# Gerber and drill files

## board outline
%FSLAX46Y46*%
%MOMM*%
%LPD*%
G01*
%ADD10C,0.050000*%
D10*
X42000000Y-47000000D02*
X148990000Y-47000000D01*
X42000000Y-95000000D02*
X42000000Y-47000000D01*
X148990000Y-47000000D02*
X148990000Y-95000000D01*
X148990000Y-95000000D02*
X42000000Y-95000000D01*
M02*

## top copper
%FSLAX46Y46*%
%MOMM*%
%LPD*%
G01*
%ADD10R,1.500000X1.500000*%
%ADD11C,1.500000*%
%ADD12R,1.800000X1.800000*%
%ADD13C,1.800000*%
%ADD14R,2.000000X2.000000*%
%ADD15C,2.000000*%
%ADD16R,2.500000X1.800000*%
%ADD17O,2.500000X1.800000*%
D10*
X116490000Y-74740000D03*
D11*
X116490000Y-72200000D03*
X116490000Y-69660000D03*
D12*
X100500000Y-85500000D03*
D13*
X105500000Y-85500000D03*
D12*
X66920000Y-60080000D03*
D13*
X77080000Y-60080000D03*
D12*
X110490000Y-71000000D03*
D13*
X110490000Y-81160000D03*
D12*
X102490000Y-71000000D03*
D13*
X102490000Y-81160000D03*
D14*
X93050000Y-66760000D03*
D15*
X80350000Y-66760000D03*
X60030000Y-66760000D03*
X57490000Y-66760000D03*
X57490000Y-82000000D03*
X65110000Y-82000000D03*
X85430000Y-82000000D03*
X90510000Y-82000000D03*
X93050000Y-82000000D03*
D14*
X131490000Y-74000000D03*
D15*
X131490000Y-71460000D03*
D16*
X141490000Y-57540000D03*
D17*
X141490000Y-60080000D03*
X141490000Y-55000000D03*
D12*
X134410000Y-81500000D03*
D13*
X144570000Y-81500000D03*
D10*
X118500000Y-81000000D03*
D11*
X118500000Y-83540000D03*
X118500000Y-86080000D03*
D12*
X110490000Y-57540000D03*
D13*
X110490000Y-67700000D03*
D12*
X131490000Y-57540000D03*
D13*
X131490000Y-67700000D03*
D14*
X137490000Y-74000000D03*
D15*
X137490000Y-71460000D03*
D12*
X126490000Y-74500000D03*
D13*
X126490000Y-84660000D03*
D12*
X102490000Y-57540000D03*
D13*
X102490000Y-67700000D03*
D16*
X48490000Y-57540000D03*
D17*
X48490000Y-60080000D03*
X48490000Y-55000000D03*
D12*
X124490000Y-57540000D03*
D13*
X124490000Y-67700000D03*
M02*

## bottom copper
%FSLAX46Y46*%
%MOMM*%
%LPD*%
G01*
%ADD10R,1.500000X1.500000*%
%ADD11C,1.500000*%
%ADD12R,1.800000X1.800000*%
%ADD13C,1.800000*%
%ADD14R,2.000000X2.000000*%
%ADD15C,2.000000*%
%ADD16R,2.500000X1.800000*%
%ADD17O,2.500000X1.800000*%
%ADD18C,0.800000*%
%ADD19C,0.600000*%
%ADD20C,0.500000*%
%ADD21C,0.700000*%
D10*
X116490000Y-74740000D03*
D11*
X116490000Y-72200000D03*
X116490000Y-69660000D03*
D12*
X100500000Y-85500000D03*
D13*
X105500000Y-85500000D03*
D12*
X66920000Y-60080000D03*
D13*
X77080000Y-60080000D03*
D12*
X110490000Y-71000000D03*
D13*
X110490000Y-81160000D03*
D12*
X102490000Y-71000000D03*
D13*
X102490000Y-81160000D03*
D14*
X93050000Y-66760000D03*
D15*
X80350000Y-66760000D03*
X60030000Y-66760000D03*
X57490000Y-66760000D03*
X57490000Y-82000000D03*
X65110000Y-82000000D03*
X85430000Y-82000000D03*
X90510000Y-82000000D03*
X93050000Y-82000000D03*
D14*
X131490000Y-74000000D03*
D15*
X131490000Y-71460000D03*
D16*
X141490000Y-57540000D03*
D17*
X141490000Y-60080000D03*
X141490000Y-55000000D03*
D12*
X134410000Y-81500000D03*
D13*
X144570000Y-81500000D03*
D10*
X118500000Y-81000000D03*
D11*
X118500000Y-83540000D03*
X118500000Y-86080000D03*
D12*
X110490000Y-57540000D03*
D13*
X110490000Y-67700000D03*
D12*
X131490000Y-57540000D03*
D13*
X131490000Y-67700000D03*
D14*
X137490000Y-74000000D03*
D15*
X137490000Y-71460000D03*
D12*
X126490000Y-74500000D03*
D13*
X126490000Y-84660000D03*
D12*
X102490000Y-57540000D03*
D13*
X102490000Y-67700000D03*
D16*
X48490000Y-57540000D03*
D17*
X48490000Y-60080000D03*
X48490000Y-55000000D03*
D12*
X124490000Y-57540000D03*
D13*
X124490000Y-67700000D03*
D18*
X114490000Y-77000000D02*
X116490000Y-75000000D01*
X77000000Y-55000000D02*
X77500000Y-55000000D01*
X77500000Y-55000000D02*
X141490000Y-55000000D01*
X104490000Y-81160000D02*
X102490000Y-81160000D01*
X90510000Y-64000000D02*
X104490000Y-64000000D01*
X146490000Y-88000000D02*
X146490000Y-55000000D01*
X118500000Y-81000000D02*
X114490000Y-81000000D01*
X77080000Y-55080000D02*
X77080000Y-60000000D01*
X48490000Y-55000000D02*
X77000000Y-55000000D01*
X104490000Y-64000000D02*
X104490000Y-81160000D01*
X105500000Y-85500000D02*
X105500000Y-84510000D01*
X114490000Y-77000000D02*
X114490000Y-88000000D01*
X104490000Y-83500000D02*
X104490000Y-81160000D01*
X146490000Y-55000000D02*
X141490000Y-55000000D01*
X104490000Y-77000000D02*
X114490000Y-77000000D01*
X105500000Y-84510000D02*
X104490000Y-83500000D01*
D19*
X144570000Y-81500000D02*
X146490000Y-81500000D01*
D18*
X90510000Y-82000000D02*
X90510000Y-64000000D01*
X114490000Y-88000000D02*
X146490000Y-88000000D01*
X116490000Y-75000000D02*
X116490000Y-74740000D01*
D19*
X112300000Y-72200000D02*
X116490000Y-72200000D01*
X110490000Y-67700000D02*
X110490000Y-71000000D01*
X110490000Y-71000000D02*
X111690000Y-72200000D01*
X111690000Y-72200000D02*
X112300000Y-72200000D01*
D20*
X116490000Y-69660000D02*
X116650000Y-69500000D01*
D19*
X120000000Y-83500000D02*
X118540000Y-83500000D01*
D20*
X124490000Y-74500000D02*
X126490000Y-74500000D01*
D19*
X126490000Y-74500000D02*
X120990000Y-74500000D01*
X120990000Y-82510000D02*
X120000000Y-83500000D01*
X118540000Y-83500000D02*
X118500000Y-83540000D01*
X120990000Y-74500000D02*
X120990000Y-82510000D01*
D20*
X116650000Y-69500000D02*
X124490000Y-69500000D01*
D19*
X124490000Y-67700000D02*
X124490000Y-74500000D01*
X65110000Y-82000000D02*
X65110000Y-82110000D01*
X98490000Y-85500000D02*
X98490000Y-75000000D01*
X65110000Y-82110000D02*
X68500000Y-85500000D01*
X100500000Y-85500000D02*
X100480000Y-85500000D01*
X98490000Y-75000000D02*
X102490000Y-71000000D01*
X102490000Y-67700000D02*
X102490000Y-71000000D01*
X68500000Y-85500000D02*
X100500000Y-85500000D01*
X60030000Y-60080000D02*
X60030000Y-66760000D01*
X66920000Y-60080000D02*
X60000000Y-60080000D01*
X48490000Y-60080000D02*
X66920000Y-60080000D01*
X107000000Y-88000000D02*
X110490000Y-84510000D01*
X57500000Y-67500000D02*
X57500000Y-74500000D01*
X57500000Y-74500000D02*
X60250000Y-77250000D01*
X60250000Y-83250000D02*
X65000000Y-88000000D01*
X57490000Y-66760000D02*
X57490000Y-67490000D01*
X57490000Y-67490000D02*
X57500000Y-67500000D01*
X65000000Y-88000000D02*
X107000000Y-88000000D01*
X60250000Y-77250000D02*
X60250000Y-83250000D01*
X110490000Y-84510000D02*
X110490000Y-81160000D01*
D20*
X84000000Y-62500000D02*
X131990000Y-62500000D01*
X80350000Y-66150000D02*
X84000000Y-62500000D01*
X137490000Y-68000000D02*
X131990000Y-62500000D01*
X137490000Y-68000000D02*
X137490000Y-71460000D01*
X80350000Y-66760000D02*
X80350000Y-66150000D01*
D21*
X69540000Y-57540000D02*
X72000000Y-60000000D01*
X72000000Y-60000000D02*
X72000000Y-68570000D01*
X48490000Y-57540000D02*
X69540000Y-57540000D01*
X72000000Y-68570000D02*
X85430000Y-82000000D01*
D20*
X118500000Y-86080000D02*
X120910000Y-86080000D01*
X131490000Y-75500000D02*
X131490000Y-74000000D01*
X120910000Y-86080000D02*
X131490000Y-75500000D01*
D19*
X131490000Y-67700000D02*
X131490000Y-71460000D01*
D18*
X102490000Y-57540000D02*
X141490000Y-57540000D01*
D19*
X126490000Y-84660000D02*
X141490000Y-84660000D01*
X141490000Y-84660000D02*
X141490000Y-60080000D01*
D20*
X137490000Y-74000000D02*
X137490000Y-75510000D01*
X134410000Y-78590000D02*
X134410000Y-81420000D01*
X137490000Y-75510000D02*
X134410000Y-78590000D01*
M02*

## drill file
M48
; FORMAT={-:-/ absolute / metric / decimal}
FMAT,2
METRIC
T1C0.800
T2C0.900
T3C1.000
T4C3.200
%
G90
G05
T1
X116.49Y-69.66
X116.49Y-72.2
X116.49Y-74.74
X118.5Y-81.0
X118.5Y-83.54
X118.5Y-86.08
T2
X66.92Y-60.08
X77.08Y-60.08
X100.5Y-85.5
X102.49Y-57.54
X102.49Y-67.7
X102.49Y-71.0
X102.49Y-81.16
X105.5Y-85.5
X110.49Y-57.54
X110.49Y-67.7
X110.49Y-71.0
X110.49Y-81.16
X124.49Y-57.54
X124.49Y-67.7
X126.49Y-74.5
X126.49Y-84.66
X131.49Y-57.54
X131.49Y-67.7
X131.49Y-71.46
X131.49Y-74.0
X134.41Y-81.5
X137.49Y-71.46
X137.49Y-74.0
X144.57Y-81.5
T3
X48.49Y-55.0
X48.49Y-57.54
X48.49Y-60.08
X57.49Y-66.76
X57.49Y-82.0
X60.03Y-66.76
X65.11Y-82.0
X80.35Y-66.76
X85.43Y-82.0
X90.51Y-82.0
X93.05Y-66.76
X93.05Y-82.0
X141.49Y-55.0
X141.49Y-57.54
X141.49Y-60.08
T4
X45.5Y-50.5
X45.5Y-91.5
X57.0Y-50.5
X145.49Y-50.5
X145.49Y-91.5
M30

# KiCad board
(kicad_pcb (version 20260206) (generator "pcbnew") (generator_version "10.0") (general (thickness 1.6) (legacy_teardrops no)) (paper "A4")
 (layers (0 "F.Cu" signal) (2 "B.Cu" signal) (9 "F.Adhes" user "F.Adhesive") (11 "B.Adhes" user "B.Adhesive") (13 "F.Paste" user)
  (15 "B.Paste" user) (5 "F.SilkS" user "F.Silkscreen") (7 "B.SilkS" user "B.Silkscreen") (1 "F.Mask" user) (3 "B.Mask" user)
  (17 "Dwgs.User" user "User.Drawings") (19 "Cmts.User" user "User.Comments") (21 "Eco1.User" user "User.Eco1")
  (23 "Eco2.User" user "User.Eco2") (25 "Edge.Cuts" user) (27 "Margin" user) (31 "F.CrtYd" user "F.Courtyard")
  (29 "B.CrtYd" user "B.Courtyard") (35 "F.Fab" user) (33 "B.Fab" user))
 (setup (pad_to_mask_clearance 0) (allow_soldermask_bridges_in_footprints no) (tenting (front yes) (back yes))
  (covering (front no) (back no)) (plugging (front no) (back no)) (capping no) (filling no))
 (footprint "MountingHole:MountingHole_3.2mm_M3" (layer "F.Cu") (at 145.49 50.5)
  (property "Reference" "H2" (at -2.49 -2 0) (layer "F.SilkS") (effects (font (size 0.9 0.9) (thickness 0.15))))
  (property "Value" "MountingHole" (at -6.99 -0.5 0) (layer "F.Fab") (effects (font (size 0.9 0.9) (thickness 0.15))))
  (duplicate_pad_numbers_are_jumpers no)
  (pad "" np_thru_hole circle (at 0 0) (size 3.2 3.2) (drill 3.2) (layers "*.Cu" "*.Mask")))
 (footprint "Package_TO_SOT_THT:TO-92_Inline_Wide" (layer "F.Cu") (at 116.49 74.74 90)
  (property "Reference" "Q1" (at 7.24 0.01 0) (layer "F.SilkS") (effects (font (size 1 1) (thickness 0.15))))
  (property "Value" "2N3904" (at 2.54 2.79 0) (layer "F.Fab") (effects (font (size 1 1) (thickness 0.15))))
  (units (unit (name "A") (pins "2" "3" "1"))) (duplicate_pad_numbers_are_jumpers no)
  (pad "1" thru_hole rect (at 0 0) (size 1.5 1.5) (drill 0.8) (layers "*.Cu" "*.Mask") (remove_unused_layers no) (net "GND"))
  (pad "2" thru_hole circle (at 2.54 0) (size 1.5 1.5) (drill 0.8) (layers "*.Cu" "*.Mask") (remove_unused_layers no) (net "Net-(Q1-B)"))
  (pad "3" thru_hole circle (at 5.08 0) (size 1.5 1.5) (drill 0.8) (layers "*.Cu" "*.Mask") (remove_unused_layers no) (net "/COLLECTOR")))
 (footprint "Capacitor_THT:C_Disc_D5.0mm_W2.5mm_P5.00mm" (layer "F.Cu") (at 100.5 85.5)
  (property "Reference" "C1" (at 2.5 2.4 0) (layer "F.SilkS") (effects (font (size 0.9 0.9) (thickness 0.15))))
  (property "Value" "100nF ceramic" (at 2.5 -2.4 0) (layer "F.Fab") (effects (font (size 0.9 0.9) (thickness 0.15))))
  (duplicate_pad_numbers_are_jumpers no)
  (pad "1" thru_hole rect (at 0 0) (size 1.8 1.8) (drill 0.9) (layers "*.Cu" "*.Mask") (remove_unused_layers no) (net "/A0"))
  (pad "2" thru_hole circle (at 5 0) (size 1.8 1.8) (drill 0.9) (layers "*.Cu" "*.Mask") (remove_unused_layers no) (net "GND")))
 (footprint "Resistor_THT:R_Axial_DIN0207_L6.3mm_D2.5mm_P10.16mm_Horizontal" (layer "F.Cu") (at 66.92 60.08)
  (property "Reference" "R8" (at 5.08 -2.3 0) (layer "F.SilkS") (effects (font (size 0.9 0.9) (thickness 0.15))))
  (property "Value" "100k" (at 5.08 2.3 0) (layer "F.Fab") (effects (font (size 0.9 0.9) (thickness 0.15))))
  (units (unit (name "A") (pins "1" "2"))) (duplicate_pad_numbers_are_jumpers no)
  (pad "1" thru_hole rect (at 0 0) (size 1.8 1.8) (drill 0.9) (layers "*.Cu" "*.Mask") (remove_unused_layers no) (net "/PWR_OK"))
  (pad "2" thru_hole circle (at 10.16 0) (size 1.8 1.8) (drill 0.9) (layers "*.Cu" "*.Mask") (remove_unused_layers no) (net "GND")))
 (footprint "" (layer "F.Cu") (at 57 50.5)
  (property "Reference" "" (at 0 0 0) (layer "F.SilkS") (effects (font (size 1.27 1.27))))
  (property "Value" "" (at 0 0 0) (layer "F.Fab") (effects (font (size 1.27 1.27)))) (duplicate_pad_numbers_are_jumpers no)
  (pad "" np_thru_hole circle (at 0 0) (size 3.2 3.2) (drill 3.2) (layers "*.Cu" "*.Mask")))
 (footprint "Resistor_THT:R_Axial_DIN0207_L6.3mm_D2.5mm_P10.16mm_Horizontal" (layer "F.Cu") (at 110.49 71 -90)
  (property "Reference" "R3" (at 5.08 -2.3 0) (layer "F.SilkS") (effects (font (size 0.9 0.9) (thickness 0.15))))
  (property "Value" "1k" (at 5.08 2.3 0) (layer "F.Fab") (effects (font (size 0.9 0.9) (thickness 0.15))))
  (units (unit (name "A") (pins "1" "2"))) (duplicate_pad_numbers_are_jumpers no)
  (pad "1" thru_hole rect (at 0 0) (size 1.8 1.8) (drill 0.9) (layers "*.Cu" "*.Mask") (remove_unused_layers no) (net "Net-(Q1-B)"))
  (pad "2" thru_hole circle (at 10.16 0) (size 1.8 1.8) (drill 0.9) (layers "*.Cu" "*.Mask") (remove_unused_layers no) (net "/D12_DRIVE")))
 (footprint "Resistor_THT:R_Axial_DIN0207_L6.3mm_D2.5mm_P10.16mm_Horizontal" (layer "F.Cu") (at 102.49 71 -90)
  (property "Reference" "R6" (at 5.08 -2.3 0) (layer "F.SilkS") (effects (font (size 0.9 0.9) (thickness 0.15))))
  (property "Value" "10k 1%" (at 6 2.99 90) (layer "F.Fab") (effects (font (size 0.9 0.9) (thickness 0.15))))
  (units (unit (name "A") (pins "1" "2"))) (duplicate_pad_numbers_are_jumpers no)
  (pad "1" thru_hole rect (at 0 0) (size 1.8 1.8) (drill 0.9) (layers "*.Cu" "*.Mask") (remove_unused_layers no) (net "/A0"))
  (pad "2" thru_hole circle (at 10.16 0) (size 1.8 1.8) (drill 0.9) (layers "*.Cu" "*.Mask") (remove_unused_layers no) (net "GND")))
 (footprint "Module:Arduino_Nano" (layer "F.Cu") (at 57.49 82 90)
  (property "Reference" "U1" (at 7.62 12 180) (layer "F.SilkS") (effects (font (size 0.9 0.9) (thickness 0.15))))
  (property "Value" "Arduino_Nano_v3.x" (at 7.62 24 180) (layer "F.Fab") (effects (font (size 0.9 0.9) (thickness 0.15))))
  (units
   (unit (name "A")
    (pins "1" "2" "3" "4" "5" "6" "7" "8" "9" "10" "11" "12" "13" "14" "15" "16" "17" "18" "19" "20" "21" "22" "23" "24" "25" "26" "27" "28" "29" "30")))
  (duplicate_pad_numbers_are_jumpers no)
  (pad "1" thru_hole rect (at 15.24 35.56 180) (size 2 2) (drill 1) (layers "*.Cu" "*.Mask") (remove_unused_layers no))
  (pad "6" thru_hole circle (at 15.24 22.86 180) (size 2 2) (drill 1) (layers "*.Cu" "*.Mask") (remove_unused_layers no) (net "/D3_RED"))
  (pad "14" thru_hole circle (at 15.24 2.54 180) (size 2 2) (drill 1) (layers "*.Cu" "*.Mask") (remove_unused_layers no) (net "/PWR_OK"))
  (pad "15" thru_hole circle (at 15.24 0 180) (size 2 2) (drill 1) (layers "*.Cu" "*.Mask") (remove_unused_layers no) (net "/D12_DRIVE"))
  (pad "16" thru_hole circle (at 0 0 180) (size 2 2) (drill 1) (layers "*.Cu" "*.Mask") (remove_unused_layers no))
  (pad "19" thru_hole circle (at 0 7.62 180) (size 2 2) (drill 1) (layers "*.Cu" "*.Mask") (remove_unused_layers no) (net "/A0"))
  (pad "27" thru_hole circle (at 0 27.94 180) (size 2 2) (drill 1) (layers "*.Cu" "*.Mask") (remove_unused_layers no) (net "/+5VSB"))
  (pad "29" thru_hole circle (at 0 33.02 180) (size 2 2) (drill 1) (layers "*.Cu" "*.Mask") (remove_unused_layers no) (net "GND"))
  (pad "30" thru_hole circle (at 0 35.56 180) (size 2 2) (drill 1) (layers "*.Cu" "*.Mask") (remove_unused_layers no)))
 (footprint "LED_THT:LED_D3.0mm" (layer "F.Cu") (at 131.49 74 90)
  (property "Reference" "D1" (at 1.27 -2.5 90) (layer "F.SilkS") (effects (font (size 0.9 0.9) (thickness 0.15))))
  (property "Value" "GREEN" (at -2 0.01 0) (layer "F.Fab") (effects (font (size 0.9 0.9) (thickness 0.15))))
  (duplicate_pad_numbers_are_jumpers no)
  (pad "1" thru_hole rect (at 0 0 90) (size 2 2) (drill 0.9) (layers "*.Cu" "*.Mask") (remove_unused_layers no) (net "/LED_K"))
  (pad "2" thru_hole circle (at 2.54 0 90) (size 2 2) (drill 0.9) (layers "*.Cu" "*.Mask") (remove_unused_layers no) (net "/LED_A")))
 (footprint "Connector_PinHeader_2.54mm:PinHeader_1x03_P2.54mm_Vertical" (layer "F.Cu") (at 141.49 55)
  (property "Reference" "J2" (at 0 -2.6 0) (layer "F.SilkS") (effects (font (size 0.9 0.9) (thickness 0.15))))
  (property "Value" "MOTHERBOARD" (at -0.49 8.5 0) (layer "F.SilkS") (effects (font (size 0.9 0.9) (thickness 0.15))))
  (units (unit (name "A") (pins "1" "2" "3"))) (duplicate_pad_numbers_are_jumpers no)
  (pad "1" thru_hole rect (at 0 2.54) (size 2.5 1.8) (drill 1) (layers "*.Cu" "*.Mask") (remove_unused_layers no) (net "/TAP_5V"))
  (pad "2" thru_hole oval (at 0 5.08) (size 2.5 1.8) (drill 1) (layers "*.Cu" "*.Mask") (remove_unused_layers no) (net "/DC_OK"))
  (pad "3" thru_hole oval (at 0 0) (size 2.5 1.8) (drill 1) (layers "*.Cu" "*.Mask") (remove_unused_layers no) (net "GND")))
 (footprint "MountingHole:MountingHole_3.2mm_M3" (layer "F.Cu") (at 45.5 91.5)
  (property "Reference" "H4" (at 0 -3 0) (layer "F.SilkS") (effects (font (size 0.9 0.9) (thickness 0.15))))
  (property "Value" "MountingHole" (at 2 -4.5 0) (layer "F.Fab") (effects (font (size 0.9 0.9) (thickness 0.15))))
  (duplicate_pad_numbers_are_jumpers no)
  (pad "" np_thru_hole circle (at 0 0) (size 3.2 3.2) (drill 3.2) (layers "*.Cu" "*.Mask")))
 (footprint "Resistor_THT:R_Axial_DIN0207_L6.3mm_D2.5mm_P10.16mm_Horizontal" (layer "F.Cu") (at 134.41 81.5)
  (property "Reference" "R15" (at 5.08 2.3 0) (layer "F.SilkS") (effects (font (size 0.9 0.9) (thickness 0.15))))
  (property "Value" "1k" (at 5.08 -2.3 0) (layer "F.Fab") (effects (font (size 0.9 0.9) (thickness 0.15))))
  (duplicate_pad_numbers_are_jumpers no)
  (pad "1" thru_hole rect (at 0 0) (size 1.8 1.8) (drill 0.9) (layers "*.Cu" "*.Mask") (remove_unused_layers no) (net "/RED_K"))
  (pad "2" thru_hole circle (at 10.16 0) (size 1.8 1.8) (drill 0.9) (layers "*.Cu" "*.Mask") (remove_unused_layers no) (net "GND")))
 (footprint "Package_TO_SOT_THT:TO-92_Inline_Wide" (layer "F.Cu") (at 118.5 81 -90)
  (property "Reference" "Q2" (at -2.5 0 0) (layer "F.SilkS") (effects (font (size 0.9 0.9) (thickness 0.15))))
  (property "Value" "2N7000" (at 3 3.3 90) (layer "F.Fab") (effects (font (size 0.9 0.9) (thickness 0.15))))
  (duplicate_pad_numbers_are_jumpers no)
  (pad "1" thru_hole rect (at 0 0) (size 1.5 1.5) (drill 0.8) (layers "*.Cu" "*.Mask") (remove_unused_layers no) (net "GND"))
  (pad "2" thru_hole circle (at 2.54 0) (size 1.5 1.5) (drill 0.8) (layers "*.Cu" "*.Mask") (remove_unused_layers no) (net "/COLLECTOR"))
  (pad "3" thru_hole circle (at 5.08 0) (size 1.5 1.5) (drill 0.8) (layers "*.Cu" "*.Mask") (remove_unused_layers no) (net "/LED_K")))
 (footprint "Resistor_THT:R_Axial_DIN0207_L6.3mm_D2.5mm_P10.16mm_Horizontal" (layer "F.Cu") (at 110.49 57.54 -90)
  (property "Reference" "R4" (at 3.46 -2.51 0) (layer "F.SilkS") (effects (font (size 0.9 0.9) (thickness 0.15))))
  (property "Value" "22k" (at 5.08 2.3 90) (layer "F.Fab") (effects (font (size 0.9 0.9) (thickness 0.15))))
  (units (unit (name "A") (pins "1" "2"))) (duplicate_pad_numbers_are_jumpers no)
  (pad "1" thru_hole rect (at 0 0 270) (size 1.8 1.8) (drill 0.9) (layers "*.Cu" "*.Mask") (remove_unused_layers no) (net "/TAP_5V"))
  (pad "2" thru_hole circle (at 10.16 0 270) (size 1.8 1.8) (drill 0.9) (layers "*.Cu" "*.Mask") (remove_unused_layers no)
   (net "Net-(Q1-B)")))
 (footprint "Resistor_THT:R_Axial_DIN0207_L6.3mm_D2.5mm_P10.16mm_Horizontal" (layer "F.Cu") (at 131.49 57.54 -90)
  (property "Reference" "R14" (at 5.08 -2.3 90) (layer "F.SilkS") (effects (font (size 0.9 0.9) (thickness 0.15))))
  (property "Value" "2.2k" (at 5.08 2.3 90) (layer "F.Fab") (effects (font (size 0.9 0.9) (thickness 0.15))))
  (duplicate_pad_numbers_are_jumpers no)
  (pad "1" thru_hole rect (at 0 0 270) (size 1.8 1.8) (drill 0.9) (layers "*.Cu" "*.Mask") (remove_unused_layers no) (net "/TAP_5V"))
  (pad "2" thru_hole circle (at 10.16 0 270) (size 1.8 1.8) (drill 0.9) (layers "*.Cu" "*.Mask") (remove_unused_layers no) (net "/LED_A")))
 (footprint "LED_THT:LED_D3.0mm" (layer "F.Cu") (at 137.49 74 90)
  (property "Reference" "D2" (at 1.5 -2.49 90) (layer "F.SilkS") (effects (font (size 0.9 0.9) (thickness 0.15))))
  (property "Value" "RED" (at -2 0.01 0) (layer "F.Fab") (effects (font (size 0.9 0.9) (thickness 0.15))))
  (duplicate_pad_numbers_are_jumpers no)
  (pad "1" thru_hole rect (at 0 0 90) (size 2 2) (drill 0.9) (layers "*.Cu" "*.Mask") (remove_unused_layers no) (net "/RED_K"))
  (pad "2" thru_hole circle (at 2.54 0 90) (size 2 2) (drill 0.9) (layers "*.Cu" "*.Mask") (remove_unused_layers no) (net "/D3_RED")))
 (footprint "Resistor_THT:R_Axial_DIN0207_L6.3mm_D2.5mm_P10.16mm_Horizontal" (layer "F.Cu") (at 126.49 74.5 -90)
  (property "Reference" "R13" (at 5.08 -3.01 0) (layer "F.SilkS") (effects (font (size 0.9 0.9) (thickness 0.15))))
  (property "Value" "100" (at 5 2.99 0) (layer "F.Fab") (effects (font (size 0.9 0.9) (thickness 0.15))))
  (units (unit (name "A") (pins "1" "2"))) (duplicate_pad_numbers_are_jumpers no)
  (pad "1" thru_hole rect (at 0 0) (size 1.8 1.8) (drill 0.9) (layers "*.Cu" "*.Mask") (remove_unused_layers no) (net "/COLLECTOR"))
  (pad "2" thru_hole circle (at 10.16 0) (size 1.8 1.8) (drill 0.9) (layers "*.Cu" "*.Mask") (remove_unused_layers no) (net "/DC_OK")))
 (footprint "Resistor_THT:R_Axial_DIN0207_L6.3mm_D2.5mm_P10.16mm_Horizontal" (layer "F.Cu") (at 102.49 57.54 -90)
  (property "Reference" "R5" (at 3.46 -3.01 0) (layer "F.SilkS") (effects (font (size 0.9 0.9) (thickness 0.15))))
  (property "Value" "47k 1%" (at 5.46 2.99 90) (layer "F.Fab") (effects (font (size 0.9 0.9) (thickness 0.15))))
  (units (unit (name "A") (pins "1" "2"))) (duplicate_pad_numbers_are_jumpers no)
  (pad "1" thru_hole rect (at 0 0 270) (size 1.8 1.8) (drill 0.9) (layers "*.Cu" "*.Mask") (remove_unused_layers no) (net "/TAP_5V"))
  (pad "2" thru_hole circle (at 10.16 0 270) (size 1.8 1.8) (drill 0.9) (layers "*.Cu" "*.Mask") (remove_unused_layers no) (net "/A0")))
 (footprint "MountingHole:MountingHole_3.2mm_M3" (layer "F.Cu") (at 145.49 91.5)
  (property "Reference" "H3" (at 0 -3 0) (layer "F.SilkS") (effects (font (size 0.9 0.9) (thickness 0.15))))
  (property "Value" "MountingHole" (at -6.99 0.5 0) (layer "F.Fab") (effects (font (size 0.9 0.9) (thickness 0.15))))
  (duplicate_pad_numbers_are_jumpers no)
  (pad "" np_thru_hole circle (at 0 0) (size 3.2 3.2) (drill 3.2) (layers "*.Cu" "*.Mask")))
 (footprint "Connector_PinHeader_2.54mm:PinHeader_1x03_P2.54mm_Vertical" (layer "F.Cu") (at 48.49 55)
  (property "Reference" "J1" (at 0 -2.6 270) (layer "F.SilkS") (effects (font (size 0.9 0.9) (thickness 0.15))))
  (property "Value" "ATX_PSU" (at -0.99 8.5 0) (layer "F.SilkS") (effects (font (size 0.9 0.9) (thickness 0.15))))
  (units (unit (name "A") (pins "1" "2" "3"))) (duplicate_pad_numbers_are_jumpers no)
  (pad "1" thru_hole rect (at 0 2.54) (size 2.5 1.8) (drill 1) (layers "*.Cu" "*.Mask") (remove_unused_layers no) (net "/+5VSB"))
  (pad "2" thru_hole oval (at 0 5.08) (size 2.5 1.8) (drill 1) (layers "*.Cu" "*.Mask") (remove_unused_layers no) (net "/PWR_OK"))
  (pad "3" thru_hole oval (at 0 0) (size 2.5 1.8) (drill 1) (layers "*.Cu" "*.Mask") (remove_unused_layers no) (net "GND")))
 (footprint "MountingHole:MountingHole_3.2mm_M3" (layer "F.Cu") (at 45.5 50.5)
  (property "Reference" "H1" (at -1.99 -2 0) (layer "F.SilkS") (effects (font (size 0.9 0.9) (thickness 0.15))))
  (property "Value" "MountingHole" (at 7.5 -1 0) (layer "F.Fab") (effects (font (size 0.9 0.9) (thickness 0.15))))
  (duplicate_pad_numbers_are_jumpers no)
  (pad "" np_thru_hole circle (at 0 0) (size 3.2 3.2) (drill 3.2) (layers "*.Cu" "*.Mask")))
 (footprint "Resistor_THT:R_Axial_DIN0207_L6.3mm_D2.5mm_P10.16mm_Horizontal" (layer "F.Cu") (at 124.49 57.54 -90)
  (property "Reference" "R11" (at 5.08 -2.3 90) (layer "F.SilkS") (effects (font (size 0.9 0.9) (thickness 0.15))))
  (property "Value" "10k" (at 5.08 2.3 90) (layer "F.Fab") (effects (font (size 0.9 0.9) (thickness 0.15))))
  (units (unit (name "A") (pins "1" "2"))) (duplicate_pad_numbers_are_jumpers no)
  (pad "1" thru_hole rect (at 0 0 270) (size 1.8 1.8) (drill 0.9) (layers "*.Cu" "*.Mask") (remove_unused_layers no) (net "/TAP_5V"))
  (pad "2" thru_hole circle (at 10.16 0 270) (size 1.8 1.8) (drill 0.9) (layers "*.Cu" "*.Mask") (remove_unused_layers no)
   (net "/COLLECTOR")))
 (gr_line (start 42 47) (end 148.99 47) (stroke (width 0.05) (type default)) (layer "Edge.Cuts"))
 (gr_line (start 42 95) (end 42 47) (stroke (width 0.05) (type default)) (layer "Edge.Cuts"))
 (gr_line (start 148.99 47) (end 148.99 95) (stroke (width 0.05) (type default)) (layer "Edge.Cuts"))
 (gr_line (start 148.99 95) (end 42 95) (stroke (width 0.05) (type default)) (layer "Edge.Cuts"))
 (segment (start 114.49 77) (end 116.49 75) (width 0.8) (layer "B.Cu") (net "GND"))
 (segment (start 77 55) (end 77.5 55) (width 0.8) (layer "B.Cu") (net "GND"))
 (segment (start 77.5 55) (end 141.49 55) (width 0.8) (layer "B.Cu") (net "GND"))
 (segment (start 104.49 81.16) (end 102.49 81.16) (width 0.8) (layer "B.Cu") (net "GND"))
 (segment (start 90.51 64) (end 104.49 64) (width 0.8) (layer "B.Cu") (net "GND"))
 (segment (start 146.49 88) (end 146.49 55) (width 0.8) (layer "B.Cu") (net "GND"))
 (segment (start 118.5 81) (end 114.49 81) (width 0.8) (layer "B.Cu") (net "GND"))
 (segment (start 77.08 55.08) (end 77.08 60) (width 0.8) (layer "B.Cu") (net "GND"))
 (segment (start 48.49 55) (end 77 55) (width 0.8) (layer "B.Cu") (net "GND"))
 (segment (start 104.49 64) (end 104.49 81.16) (width 0.8) (layer "B.Cu") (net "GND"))
 (segment (start 105.5 85.5) (end 105.5 84.51) (width 0.8) (layer "B.Cu") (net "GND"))
 (segment (start 114.49 77) (end 114.49 88) (width 0.8) (layer "B.Cu") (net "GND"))
 (segment (start 104.49 83.5) (end 104.49 81.16) (width 0.8) (layer "B.Cu") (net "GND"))
 (segment (start 146.49 55) (end 141.49 55) (width 0.8) (layer "B.Cu") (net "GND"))
 (segment (start 104.49 77) (end 114.49 77) (width 0.8) (layer "B.Cu") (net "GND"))
 (segment (start 105.5 84.51) (end 104.49 83.5) (width 0.8) (layer "B.Cu") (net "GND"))
 (segment (start 144.57 81.5) (end 146.49 81.5) (width 0.6) (layer "B.Cu") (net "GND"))
 (segment (start 90.51 82) (end 90.51 64) (width 0.8) (layer "B.Cu") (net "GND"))
 (segment (start 114.49 88) (end 146.49 88) (width 0.8) (layer "B.Cu") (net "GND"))
 (segment (start 116.49 75) (end 116.49 74.74) (width 0.8) (layer "B.Cu") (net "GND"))
 (segment (start 112.3 72.2) (end 116.49 72.2) (width 0.6) (layer "B.Cu") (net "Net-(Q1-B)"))
 (segment (start 110.49 67.7) (end 110.49 71) (width 0.6) (layer "B.Cu") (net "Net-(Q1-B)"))
 (segment (start 110.49 71) (end 111.69 72.2) (width 0.6) (layer "B.Cu") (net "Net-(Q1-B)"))
 (segment (start 111.69 72.2) (end 112.3 72.2) (width 0.6) (layer "B.Cu") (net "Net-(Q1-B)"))
 (segment (start 116.49 69.66) (end 116.65 69.5) (width 0.5) (layer "B.Cu") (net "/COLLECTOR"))
 (segment (start 120 83.5) (end 118.54 83.5) (width 0.6) (layer "B.Cu") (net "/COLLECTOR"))
 (segment (start 124.49 74.5) (end 126.49 74.5) (width 0.5) (layer "B.Cu") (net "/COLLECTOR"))
 (segment (start 126.49 74.5) (end 120.99 74.5) (width 0.6) (layer "B.Cu") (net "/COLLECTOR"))
 (segment (start 120.99 82.51) (end 120 83.5) (width 0.6) (layer "B.Cu") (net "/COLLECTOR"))
 (segment (start 118.54 83.5) (end 118.5 83.54) (width 0.6) (layer "B.Cu") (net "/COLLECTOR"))
 (segment (start 120.99 74.5) (end 120.99 82.51) (width 0.6) (layer "B.Cu") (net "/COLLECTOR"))
 (segment (start 116.65 69.5) (end 124.49 69.5) (width 0.5) (layer "B.Cu") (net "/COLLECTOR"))
 (segment (start 124.49 67.7) (end 124.49 74.5) (width 0.6) (layer "B.Cu") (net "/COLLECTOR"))
 (segment (start 65.11 82) (end 65.11 82.11) (width 0.6) (layer "B.Cu") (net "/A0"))
 (segment (start 98.49 85.5) (end 98.49 75) (width 0.6) (layer "B.Cu") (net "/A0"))
 (segment (start 65.11 82.11) (end 68.5 85.5) (width 0.6) (layer "B.Cu") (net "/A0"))
 (segment (start 100.5 85.5) (end 100.48 85.5) (width 0.6) (layer "B.Cu") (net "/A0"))
 (segment (start 98.49 75) (end 102.49 71) (width 0.6) (layer "B.Cu") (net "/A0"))
 (segment (start 102.49 67.7) (end 102.49 71) (width 0.6) (layer "B.Cu") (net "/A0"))
 (segment (start 68.5 85.5) (end 100.5 85.5) (width 0.6) (layer "B.Cu") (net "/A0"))
 (segment (start 60.03 60.08) (end 60.03 66.76) (width 0.6) (layer "B.Cu") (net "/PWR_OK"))
 (segment (start 66.92 60.08) (end 60 60.08) (width 0.6) (layer "B.Cu") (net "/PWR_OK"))
 (segment (start 48.49 60.08) (end 66.92 60.08) (width 0.6) (layer "B.Cu") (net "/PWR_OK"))
 (segment (start 107 88) (end 110.49 84.51) (width 0.6) (layer "B.Cu") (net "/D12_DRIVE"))
 (segment (start 57.5 67.5) (end 57.5 74.5) (width 0.6) (layer "B.Cu") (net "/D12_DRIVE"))
 (segment (start 57.5 74.5) (end 60.25 77.25) (width 0.6) (layer "B.Cu") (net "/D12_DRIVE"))
 (segment (start 60.25 83.25) (end 65 88) (width 0.6) (layer "B.Cu") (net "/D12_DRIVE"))
 (segment (start 57.49 66.76) (end 57.49 67.49) (width 0.6) (layer "B.Cu") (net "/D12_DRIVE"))
 (segment (start 57.49 67.49) (end 57.5 67.5) (width 0.6) (layer "B.Cu") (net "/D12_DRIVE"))
 (segment (start 65 88) (end 107 88) (width 0.6) (layer "B.Cu") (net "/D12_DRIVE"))
 (segment (start 60.25 77.25) (end 60.25 83.25) (width 0.6) (layer "B.Cu") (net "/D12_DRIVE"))
 (segment (start 110.49 84.51) (end 110.49 81.16) (width 0.6) (layer "B.Cu") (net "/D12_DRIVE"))
 (segment (start 84 62.5) (end 131.99 62.5) (width 0.5) (layer "B.Cu") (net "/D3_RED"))
 (segment (start 80.35 66.15) (end 84 62.5) (width 0.5) (layer "B.Cu") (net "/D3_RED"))
 (segment (start 137.49 68) (end 131.99 62.5) (width 0.5) (layer "B.Cu") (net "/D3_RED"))
 (segment (start 137.49 68) (end 137.49 71.46) (width 0.5) (layer "B.Cu") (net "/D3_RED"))
 (segment (start 80.35 66.76) (end 80.35 66.15) (width 0.5) (layer "B.Cu") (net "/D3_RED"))
 (segment (start 69.54 57.54) (end 72 60) (width 0.7) (layer "B.Cu") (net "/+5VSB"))
 (segment (start 72 60) (end 72 68.57) (width 0.7) (layer "B.Cu") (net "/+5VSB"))
 (segment (start 48.49 57.54) (end 69.54 57.54) (width 0.7) (layer "B.Cu") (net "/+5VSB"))
 (segment (start 72 68.57) (end 85.43 82) (width 0.7) (layer "B.Cu") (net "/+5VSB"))
 (segment (start 118.5 86.08) (end 120.91 86.08) (width 0.5) (layer "B.Cu") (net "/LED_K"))
 (segment (start 131.49 75.5) (end 131.49 74) (width 0.5) (layer "B.Cu") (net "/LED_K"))
 (segment (start 120.91 86.08) (end 131.49 75.5) (width 0.5) (layer "B.Cu") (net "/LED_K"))
 (segment (start 131.49 67.7) (end 131.49 71.46) (width 0.6) (layer "B.Cu") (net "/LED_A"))
 (segment (start 102.49 57.54) (end 141.49 57.54) (width 0.8) (layer "B.Cu") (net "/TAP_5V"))
 (segment (start 126.49 84.66) (end 141.49 84.66) (width 0.6) (layer "B.Cu") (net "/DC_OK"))
 (segment (start 141.49 84.66) (end 141.49 60.08) (width 0.6) (layer "B.Cu") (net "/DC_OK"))
 (segment (start 137.49 74) (end 137.49 75.51) (width 0.5) (layer "B.Cu") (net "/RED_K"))
 (segment (start 134.41 78.59) (end 134.41 81.42) (width 0.5) (layer "B.Cu") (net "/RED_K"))
 (segment (start 137.49 75.51) (end 134.41 78.59) (width 0.5) (layer "B.Cu") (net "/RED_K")))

